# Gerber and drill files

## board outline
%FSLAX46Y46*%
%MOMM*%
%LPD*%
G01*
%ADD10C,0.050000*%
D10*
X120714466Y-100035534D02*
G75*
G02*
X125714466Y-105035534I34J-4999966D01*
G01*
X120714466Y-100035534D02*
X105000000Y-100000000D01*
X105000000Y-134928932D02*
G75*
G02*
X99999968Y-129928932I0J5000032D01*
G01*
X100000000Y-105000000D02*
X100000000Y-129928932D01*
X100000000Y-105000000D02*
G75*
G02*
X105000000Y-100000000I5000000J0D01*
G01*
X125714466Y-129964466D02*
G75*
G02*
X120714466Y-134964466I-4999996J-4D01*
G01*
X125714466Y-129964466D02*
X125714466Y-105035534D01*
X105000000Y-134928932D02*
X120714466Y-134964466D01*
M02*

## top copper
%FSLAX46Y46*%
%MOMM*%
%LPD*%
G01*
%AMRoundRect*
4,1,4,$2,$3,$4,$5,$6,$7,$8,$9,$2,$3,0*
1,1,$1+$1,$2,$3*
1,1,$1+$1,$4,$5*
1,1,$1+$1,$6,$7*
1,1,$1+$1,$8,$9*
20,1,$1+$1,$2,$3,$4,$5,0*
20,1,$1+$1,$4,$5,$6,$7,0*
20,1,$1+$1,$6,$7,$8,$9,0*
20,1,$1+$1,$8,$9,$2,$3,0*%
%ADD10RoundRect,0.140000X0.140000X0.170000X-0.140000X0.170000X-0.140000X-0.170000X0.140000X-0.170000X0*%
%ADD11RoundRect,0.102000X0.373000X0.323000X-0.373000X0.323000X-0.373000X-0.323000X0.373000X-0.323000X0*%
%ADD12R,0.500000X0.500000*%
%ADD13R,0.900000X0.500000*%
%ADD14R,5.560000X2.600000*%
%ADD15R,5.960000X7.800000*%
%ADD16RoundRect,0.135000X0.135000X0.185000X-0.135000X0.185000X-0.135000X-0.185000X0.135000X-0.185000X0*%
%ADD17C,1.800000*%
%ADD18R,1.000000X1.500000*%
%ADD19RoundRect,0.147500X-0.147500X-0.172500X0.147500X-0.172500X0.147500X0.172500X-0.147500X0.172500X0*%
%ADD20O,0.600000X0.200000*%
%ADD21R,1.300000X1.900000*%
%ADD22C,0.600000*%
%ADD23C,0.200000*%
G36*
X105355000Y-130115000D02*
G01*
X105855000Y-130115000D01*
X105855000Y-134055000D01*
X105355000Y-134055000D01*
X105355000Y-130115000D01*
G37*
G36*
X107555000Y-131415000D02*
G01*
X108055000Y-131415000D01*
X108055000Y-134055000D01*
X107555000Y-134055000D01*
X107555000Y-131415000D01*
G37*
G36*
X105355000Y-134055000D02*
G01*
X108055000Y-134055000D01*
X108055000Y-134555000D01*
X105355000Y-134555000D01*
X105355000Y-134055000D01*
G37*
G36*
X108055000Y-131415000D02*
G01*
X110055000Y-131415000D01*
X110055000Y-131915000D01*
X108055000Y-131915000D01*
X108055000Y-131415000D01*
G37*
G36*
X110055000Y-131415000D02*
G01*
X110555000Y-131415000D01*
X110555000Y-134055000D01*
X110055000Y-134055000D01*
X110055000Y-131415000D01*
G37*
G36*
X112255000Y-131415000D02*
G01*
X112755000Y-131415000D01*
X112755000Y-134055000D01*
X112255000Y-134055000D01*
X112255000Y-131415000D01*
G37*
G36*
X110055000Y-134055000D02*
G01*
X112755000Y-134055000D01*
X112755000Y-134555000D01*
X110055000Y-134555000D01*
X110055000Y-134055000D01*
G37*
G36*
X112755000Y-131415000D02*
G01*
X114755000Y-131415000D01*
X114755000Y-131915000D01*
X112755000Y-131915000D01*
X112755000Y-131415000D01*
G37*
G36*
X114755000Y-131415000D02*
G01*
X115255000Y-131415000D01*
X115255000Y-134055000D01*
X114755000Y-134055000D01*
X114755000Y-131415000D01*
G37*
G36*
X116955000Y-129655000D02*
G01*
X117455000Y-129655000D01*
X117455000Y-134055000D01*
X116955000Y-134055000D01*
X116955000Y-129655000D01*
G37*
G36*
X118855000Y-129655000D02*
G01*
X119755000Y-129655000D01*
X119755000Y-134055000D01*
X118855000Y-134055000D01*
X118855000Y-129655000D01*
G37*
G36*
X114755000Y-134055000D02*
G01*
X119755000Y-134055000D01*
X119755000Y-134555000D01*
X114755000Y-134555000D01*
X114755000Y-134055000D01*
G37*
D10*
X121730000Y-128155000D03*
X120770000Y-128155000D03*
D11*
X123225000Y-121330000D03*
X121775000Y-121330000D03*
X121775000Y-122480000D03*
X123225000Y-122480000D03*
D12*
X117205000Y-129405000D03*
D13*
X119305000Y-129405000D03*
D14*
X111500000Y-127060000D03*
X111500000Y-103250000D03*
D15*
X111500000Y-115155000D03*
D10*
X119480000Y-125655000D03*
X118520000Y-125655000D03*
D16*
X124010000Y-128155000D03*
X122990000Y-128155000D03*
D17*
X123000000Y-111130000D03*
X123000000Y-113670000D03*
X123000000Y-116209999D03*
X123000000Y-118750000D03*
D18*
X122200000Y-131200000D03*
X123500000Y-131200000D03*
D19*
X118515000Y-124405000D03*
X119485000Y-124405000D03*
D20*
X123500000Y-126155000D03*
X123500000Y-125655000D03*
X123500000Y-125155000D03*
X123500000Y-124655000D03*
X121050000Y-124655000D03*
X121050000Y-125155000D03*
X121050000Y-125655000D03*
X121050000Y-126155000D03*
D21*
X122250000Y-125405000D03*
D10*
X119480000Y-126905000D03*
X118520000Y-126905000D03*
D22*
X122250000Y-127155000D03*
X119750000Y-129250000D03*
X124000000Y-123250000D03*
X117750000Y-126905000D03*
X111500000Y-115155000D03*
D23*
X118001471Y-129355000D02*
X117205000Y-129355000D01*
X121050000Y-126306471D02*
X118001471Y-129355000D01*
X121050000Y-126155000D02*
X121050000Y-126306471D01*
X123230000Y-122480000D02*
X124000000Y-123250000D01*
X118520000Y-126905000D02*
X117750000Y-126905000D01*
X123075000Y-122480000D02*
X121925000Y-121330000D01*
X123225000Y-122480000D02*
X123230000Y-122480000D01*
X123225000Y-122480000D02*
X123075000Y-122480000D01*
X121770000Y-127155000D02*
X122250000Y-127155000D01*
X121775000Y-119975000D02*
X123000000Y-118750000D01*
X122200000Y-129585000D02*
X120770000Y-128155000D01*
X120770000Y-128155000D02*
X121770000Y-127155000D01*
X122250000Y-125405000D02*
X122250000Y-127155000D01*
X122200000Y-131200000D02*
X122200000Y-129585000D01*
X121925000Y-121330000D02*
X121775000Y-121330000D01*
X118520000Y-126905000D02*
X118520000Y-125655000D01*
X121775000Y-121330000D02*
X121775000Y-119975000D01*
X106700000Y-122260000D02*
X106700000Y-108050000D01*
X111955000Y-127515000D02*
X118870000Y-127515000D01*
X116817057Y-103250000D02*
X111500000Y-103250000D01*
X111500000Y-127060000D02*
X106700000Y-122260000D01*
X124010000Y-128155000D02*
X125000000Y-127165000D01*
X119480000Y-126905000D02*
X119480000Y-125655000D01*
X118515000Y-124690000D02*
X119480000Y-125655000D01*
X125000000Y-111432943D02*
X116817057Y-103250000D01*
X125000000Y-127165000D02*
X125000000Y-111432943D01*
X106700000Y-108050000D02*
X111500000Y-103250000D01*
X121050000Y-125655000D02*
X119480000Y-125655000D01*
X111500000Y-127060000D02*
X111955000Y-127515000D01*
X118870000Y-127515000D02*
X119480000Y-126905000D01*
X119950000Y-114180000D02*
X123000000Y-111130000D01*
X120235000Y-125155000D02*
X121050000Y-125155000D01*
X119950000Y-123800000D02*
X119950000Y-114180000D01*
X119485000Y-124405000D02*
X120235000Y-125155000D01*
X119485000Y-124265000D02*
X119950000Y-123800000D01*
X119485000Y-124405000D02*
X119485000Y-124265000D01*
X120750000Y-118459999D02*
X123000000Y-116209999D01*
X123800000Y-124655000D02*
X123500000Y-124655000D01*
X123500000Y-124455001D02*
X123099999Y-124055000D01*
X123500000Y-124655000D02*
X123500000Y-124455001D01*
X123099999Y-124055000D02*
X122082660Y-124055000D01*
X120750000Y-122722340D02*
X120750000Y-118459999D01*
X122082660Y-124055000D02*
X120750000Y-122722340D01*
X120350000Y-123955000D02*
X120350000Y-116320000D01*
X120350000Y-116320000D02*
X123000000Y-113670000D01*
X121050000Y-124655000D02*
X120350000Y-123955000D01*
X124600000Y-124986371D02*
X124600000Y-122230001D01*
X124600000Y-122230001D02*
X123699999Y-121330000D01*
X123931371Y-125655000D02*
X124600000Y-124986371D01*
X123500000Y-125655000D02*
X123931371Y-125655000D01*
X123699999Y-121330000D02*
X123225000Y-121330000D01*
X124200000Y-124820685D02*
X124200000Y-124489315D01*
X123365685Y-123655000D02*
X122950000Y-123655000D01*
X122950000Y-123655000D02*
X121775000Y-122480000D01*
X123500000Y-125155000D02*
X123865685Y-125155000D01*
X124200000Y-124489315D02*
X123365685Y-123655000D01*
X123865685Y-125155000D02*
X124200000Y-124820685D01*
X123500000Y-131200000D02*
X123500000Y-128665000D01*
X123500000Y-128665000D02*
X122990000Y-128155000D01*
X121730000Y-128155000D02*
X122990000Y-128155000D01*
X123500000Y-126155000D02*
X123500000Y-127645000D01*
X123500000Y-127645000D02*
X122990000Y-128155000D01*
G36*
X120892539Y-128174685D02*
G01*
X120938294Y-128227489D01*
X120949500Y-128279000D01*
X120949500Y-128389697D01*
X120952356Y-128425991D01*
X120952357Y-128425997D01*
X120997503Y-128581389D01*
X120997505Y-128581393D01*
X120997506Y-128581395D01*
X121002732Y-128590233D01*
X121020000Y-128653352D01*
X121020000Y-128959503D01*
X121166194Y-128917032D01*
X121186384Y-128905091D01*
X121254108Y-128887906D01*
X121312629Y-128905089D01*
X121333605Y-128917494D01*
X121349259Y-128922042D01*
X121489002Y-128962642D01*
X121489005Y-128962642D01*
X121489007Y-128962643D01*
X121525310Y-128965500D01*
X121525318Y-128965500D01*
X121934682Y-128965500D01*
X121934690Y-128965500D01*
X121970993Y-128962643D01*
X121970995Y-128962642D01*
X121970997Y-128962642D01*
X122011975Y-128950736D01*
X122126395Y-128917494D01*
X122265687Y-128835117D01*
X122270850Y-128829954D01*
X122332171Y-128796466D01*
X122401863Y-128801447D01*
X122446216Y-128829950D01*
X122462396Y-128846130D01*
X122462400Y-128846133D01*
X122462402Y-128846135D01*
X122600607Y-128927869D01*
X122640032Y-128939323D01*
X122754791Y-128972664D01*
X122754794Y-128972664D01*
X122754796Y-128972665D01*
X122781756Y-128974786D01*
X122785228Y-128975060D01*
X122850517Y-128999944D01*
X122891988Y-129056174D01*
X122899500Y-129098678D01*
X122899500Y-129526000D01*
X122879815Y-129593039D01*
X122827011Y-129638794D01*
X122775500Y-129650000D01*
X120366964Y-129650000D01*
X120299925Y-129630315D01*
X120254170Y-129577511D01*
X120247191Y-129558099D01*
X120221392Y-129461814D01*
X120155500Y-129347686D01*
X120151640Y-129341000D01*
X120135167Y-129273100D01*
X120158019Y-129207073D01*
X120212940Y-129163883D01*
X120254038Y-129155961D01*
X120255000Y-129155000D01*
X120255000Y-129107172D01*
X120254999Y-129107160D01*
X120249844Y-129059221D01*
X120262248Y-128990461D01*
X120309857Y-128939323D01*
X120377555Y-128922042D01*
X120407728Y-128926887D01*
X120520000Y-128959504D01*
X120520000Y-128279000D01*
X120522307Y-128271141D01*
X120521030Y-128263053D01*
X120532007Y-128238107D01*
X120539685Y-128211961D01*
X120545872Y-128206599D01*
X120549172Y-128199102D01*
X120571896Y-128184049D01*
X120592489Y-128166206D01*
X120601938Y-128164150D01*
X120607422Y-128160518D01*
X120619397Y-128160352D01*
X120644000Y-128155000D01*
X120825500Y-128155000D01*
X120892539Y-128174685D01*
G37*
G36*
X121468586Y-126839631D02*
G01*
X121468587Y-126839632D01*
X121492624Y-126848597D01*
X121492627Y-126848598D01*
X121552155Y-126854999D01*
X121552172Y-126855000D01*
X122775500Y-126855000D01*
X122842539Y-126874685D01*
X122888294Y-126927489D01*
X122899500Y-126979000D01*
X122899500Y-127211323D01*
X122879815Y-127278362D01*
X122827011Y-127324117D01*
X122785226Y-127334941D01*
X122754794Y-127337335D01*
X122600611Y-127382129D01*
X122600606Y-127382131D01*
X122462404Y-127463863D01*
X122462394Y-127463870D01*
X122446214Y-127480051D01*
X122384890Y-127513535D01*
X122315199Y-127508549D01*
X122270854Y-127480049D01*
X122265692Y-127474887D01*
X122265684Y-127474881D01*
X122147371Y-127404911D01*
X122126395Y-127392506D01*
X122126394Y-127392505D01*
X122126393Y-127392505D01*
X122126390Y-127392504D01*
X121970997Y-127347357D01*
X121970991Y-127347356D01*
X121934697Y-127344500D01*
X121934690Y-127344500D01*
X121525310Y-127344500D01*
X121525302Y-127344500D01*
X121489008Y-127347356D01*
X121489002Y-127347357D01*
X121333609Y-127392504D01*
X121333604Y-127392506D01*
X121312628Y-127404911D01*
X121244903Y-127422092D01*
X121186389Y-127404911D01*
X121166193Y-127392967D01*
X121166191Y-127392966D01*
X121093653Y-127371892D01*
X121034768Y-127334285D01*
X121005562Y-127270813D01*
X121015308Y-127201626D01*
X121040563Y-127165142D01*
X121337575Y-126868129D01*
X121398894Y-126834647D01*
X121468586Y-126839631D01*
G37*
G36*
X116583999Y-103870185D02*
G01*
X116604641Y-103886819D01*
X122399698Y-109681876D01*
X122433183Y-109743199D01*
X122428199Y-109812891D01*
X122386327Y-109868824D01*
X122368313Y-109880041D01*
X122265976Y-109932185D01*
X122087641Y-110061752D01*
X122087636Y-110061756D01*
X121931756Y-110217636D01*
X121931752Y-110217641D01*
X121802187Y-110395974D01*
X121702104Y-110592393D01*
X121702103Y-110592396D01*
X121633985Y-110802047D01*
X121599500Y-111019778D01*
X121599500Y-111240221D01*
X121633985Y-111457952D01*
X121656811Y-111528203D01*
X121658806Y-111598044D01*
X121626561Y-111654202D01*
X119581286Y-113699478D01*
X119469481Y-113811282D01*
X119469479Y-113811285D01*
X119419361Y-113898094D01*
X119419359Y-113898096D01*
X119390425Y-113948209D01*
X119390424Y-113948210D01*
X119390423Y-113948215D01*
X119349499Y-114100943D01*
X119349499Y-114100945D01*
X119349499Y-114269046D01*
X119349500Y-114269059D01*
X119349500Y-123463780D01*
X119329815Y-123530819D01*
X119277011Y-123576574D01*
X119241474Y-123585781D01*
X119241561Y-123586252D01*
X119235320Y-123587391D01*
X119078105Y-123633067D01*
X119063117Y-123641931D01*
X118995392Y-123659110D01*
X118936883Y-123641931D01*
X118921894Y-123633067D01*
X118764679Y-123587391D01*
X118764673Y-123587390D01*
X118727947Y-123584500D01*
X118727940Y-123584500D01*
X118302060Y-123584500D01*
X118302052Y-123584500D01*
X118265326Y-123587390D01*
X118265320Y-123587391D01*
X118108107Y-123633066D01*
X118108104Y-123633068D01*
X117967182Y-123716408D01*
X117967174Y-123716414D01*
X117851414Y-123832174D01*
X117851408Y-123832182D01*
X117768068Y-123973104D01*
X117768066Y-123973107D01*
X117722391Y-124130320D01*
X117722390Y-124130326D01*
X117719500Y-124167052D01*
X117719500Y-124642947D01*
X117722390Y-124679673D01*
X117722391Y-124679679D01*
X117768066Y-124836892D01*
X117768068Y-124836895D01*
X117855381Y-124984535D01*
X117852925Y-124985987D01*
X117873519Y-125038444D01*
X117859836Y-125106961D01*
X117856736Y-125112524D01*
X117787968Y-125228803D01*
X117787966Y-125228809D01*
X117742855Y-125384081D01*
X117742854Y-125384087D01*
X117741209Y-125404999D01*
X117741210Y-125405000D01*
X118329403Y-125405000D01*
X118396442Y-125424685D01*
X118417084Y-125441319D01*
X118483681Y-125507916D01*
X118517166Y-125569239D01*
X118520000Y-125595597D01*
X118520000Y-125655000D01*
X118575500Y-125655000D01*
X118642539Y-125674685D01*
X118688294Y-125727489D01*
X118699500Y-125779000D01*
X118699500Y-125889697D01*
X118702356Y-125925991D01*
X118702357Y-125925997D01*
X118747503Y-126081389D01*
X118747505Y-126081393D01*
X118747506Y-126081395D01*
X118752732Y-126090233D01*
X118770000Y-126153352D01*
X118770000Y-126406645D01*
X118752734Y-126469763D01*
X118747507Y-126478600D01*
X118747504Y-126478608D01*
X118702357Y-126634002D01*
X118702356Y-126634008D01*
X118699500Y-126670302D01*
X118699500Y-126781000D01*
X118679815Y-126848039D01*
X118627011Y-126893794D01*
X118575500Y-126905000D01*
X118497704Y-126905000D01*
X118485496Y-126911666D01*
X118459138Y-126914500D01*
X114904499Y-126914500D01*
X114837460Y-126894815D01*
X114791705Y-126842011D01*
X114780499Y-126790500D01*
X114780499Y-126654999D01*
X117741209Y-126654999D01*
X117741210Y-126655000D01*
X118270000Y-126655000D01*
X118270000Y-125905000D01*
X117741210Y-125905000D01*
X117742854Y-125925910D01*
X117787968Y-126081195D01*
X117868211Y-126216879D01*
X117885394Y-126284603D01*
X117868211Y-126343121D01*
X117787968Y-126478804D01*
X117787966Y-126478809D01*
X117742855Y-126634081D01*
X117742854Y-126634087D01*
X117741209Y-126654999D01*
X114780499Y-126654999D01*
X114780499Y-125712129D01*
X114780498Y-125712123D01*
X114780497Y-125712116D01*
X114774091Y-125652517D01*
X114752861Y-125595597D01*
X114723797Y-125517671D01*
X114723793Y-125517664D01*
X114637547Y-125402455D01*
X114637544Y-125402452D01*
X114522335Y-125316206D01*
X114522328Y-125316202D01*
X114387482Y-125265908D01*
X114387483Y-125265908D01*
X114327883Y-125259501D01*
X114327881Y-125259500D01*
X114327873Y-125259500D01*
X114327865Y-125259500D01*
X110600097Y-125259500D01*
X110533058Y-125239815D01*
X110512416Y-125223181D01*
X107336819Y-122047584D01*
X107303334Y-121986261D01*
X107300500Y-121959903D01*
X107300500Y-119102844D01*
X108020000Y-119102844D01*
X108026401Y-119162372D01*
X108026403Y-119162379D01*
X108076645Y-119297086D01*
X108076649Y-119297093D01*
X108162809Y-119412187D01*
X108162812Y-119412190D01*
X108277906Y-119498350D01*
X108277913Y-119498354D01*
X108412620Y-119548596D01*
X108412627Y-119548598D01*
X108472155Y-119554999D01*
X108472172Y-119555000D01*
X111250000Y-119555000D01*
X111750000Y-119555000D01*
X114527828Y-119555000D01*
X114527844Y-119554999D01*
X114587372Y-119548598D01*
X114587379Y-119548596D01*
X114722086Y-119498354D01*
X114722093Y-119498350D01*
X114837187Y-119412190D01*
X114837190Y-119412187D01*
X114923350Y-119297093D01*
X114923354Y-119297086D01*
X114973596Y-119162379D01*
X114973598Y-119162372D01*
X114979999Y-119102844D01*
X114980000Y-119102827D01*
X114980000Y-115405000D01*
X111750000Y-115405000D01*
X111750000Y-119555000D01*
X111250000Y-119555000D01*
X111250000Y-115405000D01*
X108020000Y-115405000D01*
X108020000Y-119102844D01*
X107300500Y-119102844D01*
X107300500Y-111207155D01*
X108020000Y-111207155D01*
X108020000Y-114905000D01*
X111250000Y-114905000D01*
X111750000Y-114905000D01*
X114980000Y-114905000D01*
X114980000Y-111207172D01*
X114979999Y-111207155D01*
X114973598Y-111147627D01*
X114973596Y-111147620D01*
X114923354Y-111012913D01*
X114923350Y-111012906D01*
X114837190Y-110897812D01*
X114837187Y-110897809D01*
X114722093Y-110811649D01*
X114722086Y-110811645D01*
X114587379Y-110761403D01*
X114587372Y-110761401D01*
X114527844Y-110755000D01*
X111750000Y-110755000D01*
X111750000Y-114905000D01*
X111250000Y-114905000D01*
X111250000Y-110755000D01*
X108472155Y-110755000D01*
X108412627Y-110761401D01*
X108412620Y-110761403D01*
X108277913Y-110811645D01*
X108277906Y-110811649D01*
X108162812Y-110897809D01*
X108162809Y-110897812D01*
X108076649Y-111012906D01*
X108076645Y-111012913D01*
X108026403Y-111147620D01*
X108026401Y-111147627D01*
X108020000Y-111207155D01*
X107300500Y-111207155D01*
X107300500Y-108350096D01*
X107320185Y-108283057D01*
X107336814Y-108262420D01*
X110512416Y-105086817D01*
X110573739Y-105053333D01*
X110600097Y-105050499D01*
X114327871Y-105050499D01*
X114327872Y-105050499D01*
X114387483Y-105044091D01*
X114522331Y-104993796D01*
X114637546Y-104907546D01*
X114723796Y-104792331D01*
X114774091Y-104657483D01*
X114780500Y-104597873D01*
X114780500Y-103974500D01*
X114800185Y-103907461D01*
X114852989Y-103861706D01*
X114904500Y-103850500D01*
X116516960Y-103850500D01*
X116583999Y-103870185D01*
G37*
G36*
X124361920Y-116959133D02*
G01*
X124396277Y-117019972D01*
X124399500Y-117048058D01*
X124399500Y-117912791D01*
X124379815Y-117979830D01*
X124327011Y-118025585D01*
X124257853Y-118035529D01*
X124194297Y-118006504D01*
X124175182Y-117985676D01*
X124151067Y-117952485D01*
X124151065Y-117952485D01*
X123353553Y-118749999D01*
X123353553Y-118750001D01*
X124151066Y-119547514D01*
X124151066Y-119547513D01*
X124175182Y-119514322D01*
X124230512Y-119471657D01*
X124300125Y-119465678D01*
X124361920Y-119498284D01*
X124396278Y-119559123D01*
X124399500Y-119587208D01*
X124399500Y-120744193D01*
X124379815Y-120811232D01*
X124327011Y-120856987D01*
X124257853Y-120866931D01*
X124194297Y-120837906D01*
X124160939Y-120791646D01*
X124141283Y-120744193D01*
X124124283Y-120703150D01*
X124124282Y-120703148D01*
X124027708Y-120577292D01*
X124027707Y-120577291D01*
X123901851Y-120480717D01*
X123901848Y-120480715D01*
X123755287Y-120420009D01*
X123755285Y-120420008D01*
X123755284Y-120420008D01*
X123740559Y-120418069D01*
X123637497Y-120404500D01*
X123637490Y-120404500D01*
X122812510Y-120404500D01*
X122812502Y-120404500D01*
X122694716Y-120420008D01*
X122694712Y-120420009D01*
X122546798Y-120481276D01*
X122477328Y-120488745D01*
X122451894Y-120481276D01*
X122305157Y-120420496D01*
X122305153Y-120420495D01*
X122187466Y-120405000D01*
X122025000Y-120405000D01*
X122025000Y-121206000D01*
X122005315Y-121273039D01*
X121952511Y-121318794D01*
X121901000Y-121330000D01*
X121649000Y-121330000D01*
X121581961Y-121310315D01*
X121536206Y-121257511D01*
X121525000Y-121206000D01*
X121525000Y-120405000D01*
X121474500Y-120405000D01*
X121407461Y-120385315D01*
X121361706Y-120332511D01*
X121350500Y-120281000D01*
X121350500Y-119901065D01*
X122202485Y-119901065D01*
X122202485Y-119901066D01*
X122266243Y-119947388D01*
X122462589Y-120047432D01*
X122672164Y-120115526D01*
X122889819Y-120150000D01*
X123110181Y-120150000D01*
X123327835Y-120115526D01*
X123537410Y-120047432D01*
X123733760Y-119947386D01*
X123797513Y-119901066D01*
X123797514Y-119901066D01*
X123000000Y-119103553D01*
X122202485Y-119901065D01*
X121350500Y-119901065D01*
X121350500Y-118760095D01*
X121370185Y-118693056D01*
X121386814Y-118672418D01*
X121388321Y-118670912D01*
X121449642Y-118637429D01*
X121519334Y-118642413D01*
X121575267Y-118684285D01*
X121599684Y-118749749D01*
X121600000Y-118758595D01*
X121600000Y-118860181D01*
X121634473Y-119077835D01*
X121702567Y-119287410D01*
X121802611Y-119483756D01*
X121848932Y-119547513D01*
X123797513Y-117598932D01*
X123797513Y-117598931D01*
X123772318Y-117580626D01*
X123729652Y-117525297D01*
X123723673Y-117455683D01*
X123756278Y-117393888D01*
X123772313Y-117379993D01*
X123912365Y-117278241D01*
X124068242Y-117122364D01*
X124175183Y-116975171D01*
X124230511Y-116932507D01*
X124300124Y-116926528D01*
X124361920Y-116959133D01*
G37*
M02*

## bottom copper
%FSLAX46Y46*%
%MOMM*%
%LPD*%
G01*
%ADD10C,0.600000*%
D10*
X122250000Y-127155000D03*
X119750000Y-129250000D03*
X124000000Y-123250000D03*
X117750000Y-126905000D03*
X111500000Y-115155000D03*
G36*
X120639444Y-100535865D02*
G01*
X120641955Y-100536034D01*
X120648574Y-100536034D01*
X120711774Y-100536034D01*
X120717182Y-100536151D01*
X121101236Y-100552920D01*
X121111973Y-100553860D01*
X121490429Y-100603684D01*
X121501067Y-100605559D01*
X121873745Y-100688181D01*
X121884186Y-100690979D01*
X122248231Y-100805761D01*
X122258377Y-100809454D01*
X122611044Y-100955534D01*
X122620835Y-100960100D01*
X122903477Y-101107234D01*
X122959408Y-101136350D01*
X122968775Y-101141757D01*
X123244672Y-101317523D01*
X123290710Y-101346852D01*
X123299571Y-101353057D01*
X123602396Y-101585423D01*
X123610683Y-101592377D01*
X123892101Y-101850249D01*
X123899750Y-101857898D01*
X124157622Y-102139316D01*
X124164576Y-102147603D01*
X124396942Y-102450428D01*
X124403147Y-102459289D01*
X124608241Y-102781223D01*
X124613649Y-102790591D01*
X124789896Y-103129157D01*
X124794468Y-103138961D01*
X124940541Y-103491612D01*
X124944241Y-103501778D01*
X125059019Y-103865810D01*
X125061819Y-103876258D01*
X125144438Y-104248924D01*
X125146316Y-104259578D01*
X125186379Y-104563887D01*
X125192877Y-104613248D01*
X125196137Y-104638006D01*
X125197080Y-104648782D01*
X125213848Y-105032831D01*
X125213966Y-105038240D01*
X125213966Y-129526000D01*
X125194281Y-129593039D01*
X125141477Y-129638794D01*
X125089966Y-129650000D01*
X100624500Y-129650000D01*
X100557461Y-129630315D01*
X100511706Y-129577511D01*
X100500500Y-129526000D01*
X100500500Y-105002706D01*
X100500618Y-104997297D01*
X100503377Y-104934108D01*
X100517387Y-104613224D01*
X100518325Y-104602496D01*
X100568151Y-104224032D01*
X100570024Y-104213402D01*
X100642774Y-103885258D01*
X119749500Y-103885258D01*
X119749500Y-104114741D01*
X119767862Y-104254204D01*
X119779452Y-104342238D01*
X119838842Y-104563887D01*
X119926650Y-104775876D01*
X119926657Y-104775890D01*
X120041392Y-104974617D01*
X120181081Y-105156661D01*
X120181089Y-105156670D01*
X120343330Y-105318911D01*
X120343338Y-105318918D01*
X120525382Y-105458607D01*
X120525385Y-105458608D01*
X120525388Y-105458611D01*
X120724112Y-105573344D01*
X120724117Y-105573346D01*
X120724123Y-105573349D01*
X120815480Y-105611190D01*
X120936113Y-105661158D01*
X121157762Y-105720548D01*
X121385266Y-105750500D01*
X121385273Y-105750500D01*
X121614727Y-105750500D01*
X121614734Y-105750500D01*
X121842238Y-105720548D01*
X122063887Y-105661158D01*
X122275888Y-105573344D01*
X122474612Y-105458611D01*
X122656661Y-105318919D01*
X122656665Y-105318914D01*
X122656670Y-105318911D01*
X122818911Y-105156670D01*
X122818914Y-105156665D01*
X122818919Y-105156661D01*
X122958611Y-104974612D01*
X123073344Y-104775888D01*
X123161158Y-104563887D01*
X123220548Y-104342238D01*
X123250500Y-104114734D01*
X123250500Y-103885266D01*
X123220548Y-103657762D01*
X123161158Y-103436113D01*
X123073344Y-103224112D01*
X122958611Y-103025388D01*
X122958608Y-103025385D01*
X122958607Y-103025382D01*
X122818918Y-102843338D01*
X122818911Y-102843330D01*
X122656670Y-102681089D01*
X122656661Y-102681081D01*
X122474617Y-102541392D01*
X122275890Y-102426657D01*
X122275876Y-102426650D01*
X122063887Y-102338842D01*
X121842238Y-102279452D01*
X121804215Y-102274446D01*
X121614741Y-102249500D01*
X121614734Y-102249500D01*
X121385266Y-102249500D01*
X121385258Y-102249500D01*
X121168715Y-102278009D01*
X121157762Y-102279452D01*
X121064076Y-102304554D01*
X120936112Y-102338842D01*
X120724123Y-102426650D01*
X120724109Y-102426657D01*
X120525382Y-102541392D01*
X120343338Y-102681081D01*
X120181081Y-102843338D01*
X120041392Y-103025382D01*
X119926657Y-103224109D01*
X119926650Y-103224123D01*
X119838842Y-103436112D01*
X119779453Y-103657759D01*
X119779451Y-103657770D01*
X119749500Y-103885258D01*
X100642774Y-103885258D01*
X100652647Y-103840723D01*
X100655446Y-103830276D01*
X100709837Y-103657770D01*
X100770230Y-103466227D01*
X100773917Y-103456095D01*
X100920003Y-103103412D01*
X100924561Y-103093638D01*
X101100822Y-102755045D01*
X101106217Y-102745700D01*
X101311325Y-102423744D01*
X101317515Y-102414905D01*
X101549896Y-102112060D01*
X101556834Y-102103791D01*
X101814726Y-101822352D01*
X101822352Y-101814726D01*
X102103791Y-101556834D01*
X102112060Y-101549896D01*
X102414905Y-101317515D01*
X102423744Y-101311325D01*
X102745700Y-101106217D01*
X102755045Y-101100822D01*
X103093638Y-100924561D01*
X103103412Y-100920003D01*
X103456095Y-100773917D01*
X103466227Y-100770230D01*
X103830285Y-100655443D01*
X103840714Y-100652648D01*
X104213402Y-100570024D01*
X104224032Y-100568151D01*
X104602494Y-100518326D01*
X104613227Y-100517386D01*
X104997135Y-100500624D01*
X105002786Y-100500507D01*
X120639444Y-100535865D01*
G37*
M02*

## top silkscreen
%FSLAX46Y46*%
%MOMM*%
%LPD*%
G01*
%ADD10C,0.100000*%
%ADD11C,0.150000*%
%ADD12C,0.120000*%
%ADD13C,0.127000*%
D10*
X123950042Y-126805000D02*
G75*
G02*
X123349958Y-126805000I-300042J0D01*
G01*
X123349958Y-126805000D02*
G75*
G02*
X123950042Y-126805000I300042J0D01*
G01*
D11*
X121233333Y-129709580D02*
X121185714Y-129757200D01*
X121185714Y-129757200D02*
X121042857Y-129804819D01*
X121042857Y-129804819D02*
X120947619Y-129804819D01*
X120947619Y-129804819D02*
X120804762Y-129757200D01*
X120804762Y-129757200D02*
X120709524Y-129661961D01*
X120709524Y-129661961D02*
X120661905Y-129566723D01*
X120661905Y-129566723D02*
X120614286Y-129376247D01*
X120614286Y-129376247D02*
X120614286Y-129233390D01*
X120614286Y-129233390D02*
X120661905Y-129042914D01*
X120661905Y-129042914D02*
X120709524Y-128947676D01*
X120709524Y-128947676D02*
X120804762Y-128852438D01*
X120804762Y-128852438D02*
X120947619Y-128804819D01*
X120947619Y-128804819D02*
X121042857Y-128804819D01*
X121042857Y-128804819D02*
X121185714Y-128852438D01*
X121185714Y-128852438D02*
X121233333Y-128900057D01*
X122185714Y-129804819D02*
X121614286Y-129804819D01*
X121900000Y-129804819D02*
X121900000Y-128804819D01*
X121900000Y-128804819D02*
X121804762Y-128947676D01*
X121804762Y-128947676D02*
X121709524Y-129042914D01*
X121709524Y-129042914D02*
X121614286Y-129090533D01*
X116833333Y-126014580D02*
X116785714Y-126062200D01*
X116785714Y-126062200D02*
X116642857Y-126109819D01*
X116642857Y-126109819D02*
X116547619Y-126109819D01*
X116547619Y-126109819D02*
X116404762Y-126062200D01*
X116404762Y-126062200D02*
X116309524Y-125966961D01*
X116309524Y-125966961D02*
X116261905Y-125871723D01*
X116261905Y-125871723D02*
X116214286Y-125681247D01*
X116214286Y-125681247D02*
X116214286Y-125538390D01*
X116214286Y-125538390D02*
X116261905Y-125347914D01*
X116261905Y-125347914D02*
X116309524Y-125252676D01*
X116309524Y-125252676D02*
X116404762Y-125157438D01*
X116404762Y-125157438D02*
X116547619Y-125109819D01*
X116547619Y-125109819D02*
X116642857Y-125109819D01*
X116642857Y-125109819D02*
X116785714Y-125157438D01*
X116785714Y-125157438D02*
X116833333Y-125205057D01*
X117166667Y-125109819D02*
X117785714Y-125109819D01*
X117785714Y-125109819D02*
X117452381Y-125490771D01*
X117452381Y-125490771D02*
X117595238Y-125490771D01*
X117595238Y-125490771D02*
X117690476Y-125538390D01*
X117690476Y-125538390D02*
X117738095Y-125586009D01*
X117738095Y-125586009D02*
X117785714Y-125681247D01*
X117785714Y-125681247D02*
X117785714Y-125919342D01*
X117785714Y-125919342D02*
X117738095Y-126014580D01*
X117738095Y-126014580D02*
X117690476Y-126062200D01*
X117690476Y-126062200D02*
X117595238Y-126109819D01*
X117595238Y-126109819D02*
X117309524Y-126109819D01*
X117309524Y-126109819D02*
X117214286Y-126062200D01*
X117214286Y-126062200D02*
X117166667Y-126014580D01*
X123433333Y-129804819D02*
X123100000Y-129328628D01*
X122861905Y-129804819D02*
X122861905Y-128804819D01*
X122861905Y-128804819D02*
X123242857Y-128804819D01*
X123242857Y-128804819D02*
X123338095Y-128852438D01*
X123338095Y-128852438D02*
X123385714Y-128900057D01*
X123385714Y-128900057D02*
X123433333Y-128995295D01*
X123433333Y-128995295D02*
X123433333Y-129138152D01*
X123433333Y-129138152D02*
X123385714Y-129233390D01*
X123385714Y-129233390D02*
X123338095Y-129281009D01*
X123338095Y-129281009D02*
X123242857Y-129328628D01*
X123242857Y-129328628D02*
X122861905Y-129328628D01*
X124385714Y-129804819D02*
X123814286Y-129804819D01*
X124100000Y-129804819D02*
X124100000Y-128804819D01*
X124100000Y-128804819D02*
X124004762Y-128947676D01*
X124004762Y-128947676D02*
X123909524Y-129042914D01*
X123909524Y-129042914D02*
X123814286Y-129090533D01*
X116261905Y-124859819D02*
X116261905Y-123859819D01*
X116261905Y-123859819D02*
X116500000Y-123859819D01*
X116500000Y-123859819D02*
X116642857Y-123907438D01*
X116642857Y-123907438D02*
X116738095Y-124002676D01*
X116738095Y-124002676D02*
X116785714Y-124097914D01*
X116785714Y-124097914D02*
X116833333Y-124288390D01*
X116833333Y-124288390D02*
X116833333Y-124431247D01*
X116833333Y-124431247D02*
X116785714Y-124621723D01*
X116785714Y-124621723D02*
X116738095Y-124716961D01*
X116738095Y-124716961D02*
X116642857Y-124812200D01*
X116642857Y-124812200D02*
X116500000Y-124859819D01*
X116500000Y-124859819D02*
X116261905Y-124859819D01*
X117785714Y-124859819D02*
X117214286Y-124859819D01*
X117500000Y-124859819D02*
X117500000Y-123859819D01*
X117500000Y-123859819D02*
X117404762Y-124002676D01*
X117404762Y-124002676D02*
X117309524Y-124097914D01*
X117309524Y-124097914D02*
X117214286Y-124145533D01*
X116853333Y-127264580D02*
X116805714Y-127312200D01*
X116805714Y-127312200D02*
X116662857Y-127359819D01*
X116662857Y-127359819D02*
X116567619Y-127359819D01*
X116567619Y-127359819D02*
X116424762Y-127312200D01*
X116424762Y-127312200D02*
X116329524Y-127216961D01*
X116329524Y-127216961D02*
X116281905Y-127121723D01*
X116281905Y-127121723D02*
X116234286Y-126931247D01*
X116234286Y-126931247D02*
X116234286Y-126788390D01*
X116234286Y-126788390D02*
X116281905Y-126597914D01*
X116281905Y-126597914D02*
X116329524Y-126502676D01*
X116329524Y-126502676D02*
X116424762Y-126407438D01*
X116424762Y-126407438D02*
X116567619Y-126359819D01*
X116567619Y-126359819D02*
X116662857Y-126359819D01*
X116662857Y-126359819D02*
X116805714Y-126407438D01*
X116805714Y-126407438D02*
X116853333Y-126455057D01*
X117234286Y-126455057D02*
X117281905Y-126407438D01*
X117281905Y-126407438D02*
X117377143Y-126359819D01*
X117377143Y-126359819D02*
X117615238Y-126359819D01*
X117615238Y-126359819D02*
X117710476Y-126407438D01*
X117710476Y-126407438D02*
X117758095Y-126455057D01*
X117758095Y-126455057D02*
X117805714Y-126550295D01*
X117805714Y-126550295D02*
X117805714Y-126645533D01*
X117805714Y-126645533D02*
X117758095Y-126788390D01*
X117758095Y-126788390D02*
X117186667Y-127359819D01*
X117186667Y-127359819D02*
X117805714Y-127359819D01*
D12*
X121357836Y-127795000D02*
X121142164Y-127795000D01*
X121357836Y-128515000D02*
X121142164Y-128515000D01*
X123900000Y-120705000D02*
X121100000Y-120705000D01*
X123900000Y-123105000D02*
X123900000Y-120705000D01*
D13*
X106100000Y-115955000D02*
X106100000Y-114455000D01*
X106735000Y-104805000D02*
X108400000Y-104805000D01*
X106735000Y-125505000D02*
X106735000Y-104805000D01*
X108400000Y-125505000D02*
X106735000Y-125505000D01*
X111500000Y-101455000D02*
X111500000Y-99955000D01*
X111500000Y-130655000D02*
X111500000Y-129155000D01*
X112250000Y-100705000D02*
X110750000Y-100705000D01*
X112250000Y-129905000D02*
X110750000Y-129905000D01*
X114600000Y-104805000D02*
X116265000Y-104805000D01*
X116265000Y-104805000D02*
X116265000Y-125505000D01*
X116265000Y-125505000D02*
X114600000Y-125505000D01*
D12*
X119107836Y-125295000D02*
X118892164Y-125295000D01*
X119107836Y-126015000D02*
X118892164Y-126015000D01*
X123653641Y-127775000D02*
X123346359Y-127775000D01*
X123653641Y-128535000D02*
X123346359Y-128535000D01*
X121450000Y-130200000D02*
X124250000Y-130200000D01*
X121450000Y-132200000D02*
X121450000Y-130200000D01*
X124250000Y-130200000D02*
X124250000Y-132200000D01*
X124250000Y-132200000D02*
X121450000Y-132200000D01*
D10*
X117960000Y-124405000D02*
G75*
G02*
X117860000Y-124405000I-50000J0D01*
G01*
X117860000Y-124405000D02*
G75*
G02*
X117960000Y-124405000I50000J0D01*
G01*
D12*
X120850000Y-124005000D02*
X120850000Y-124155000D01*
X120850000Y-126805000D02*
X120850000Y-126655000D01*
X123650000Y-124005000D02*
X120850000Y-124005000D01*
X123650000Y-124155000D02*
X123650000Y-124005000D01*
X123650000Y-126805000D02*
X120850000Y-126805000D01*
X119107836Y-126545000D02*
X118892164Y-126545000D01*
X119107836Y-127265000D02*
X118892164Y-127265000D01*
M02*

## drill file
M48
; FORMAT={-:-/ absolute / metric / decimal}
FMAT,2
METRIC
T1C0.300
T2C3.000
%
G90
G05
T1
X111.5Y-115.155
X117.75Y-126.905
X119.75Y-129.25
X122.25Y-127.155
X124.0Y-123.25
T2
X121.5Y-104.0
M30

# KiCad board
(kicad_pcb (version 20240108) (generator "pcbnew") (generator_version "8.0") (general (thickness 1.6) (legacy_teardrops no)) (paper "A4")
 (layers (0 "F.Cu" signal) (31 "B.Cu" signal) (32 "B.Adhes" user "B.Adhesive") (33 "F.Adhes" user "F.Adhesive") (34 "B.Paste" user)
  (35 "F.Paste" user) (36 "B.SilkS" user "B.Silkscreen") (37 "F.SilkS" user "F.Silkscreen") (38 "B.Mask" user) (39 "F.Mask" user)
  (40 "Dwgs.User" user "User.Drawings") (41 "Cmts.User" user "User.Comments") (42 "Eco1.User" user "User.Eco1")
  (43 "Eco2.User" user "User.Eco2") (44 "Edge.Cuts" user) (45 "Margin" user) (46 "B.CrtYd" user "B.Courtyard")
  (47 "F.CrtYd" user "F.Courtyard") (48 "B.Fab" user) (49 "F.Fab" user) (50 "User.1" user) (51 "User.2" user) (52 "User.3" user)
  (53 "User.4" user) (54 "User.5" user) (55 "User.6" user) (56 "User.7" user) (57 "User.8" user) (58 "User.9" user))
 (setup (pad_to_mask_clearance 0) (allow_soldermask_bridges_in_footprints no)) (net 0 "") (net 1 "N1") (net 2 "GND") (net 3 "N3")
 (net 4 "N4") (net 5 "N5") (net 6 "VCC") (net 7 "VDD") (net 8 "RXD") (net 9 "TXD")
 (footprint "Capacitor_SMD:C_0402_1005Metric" (layer "F.Cu") (at 121.25 128.155 180)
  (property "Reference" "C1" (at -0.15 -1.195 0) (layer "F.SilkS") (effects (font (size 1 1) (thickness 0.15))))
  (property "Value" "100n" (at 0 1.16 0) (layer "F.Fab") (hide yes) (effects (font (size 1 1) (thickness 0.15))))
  (fp_line (start -0.107836 0.36) (end 0.107836 0.36) (stroke (width 0.12) (type solid)) (layer "F.SilkS"))
  (fp_line (start -0.107836 -0.36) (end 0.107836 -0.36) (stroke (width 0.12) (type solid)) (layer "F.SilkS"))
  (pad "1" smd roundrect (at -0.48 0 180) (size 0.56 0.62) (layers "F.Cu" "F.Paste" "F.Mask") (roundrect_rratio 0.25) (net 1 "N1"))
  (pad "2" smd roundrect (at 0.48 0 180) (size 0.56 0.62) (layers "F.Cu" "F.Paste" "F.Mask") (roundrect_rratio 0.25) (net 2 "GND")))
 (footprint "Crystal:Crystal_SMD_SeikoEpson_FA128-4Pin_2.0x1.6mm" (layer "F.Cu") (at 122.5 121.905 180)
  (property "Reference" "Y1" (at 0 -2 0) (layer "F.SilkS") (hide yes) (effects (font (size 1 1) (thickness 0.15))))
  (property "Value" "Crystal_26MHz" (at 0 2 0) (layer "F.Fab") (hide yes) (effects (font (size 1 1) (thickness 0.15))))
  (fp_line (start -1.4 1.2) (end 1.4 1.2) (stroke (width 0.12) (type solid)) (layer "F.SilkS"))
  (fp_line (start -1.4 -1.2) (end -1.4 1.2) (stroke (width 0.12) (type solid)) (layer "F.SilkS"))
  (pad "1" smd roundrect (at -0.725 0.575 180) (size 0.95 0.85) (layers "F.Cu" "F.Paste" "F.Mask") (roundrect_rratio 0.12) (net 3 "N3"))
  (pad "2" smd roundrect (at 0.725 0.575 180) (size 0.95 0.85) (layers "F.Cu" "F.Paste" "F.Mask") (roundrect_rratio 0.12) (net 2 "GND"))
  (pad "3" smd roundrect (at 0.725 -0.575 180) (size 0.95 0.85) (layers "F.Cu" "F.Paste" "F.Mask") (roundrect_rratio 0.12) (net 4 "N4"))
  (pad "4" smd roundrect (at -0.725 -0.575 180) (size 0.95 0.85) (layers "F.Cu" "F.Paste" "F.Mask") (roundrect_rratio 0.12) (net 2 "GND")))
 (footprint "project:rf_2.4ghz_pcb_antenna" (layer "F.Cu") (at 120.255 134.855 180)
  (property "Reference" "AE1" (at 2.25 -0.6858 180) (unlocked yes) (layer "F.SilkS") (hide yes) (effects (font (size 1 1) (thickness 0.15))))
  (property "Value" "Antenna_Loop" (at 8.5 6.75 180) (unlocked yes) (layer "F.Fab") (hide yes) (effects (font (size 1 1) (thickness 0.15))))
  (fp_rect (start 14.4 0.8) (end 14.9 4.74) (stroke (width 0) (type solid)) (fill solid) (layer "F.Cu"))
  (fp_rect (start 12.2 0.8) (end 12.7 3.44) (stroke (width 0) (type default)) (fill solid) (layer "F.Cu"))
  (fp_rect (start 12.2 0.3) (end 14.9 0.8) (stroke (width 0) (type default)) (fill solid) (layer "F.Cu"))
  (fp_rect (start 10.2 2.94) (end 12.2 3.44) (stroke (width 0) (type default)) (fill solid) (layer "F.Cu"))
  (fp_rect (start 9.7 0.8) (end 10.2 3.44) (stroke (width 0) (type default)) (fill solid) (layer "F.Cu"))
  (fp_rect (start 7.5 0.8) (end 8 3.44) (stroke (width 0) (type default)) (fill solid) (layer "F.Cu"))
  (fp_rect (start 7.5 0.3) (end 10.2 0.8) (stroke (width 0) (type default)) (fill solid) (layer "F.Cu"))
  (fp_rect (start 5.5 2.94) (end 7.5 3.44) (stroke (width 0) (type default)) (fill solid) (layer "F.Cu"))
  (fp_rect (start 5 0.8) (end 5.5 3.44) (stroke (width 0) (type default)) (fill solid) (layer "F.Cu"))
  (fp_rect (start 2.8 0.8) (end 3.3 5.2) (stroke (width 0) (type default)) (fill solid) (layer "F.Cu"))
  (fp_rect (start 0.5 0.8) (end 1.4 5.2) (stroke (width 0) (type solid)) (fill solid) (layer "F.Cu"))
  (fp_rect (start 0.5 0.3) (end 5.5 0.8) (stroke (width 0) (type default)) (fill solid) (layer "F.Cu"))
  (pad "1" smd rect (at 3.05 5.45 180) (size 0.5 0.5) (layers "F.Cu" "F.Paste" "F.Mask") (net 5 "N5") (solder_mask_margin 0.102))
  (pad "2" smd rect (at 0.95 5.45 270) (size 0.5 0.9) (layers "F.Cu" "F.Paste" "F.Mask") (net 2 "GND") (solder_mask_margin 0.102))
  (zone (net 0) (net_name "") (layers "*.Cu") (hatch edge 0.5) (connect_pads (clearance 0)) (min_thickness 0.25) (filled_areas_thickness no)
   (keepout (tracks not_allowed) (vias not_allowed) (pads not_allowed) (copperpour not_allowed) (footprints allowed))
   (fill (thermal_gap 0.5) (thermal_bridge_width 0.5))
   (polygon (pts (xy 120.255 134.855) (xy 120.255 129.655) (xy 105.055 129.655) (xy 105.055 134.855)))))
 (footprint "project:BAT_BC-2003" (layer "F.Cu") (at 111.5 115.155 90)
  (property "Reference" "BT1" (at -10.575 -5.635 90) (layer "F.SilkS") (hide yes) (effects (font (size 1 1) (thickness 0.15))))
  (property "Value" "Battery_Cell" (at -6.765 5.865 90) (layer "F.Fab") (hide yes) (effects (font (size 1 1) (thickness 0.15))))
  (fp_line (start -0.8 -5.4) (end 0.7 -5.4) (stroke (width 0.127) (type solid)) (layer "F.SilkS"))
  (fp_line (start 10.35 -4.765) (end 10.35 -3.1) (stroke (width 0.127) (type solid)) (layer "F.SilkS"))
  (fp_line (start -10.35 -4.765) (end 10.35 -4.765) (stroke (width 0.127) (type solid)) (layer "F.SilkS"))
  (fp_line (start -10.35 -3.1) (end -10.35 -4.765) (stroke (width 0.127) (type solid)) (layer "F.SilkS"))
  (fp_line (start 13.7 0) (end 15.2 0) (stroke (width 0.127) (type solid)) (layer "F.SilkS"))
  (fp_line (start -15.5 0) (end -14 0) (stroke (width 0.127) (type solid)) (layer "F.SilkS"))
  (fp_line (start 14.45 0.75) (end 14.45 -0.75) (stroke (width 0.127) (type solid)) (layer "F.SilkS"))
  (fp_line (start -14.75 0.75) (end -14.75 -0.75) (stroke (width 0.127) (type solid)) (layer "F.SilkS"))
  (fp_line (start 10.35 3.1) (end 10.35 4.765) (stroke (width 0.127) (type solid)) (layer "F.SilkS"))
  (fp_line (start 10.35 4.765) (end -10.35 4.765) (stroke (width 0.127) (type solid)) (layer "F.SilkS"))
  (fp_line (start -10.35 4.765) (end -10.35 3.1) (stroke (width 0.127) (type solid)) (layer "F.SilkS"))
  (pad "1" smd rect (at -11.905 0 90) (size 2.6 5.56) (layers "F.Cu" "F.Paste" "F.Mask") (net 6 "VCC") (solder_mask_margin 0.102))
  (pad "1" smd rect (at 11.905 0 90) (size 2.6 5.56) (layers "F.Cu" "F.Paste" "F.Mask") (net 6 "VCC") (solder_mask_margin 0.102))
  (pad "2" smd rect (at 0 0 90) (size 7.8 5.96) (layers "F.Cu" "F.Mask") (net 2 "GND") (solder_mask_margin 0.102)))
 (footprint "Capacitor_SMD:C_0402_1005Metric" (layer "F.Cu") (at 119 125.655 180)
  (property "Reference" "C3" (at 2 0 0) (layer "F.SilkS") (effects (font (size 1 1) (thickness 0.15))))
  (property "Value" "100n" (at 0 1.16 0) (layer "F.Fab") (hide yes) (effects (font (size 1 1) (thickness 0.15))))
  (fp_line (start -0.107836 0.36) (end 0.107836 0.36) (stroke (width 0.12) (type solid)) (layer "F.SilkS"))
  (fp_line (start -0.107836 -0.36) (end 0.107836 -0.36) (stroke (width 0.12) (type solid)) (layer "F.SilkS"))
  (pad "1" smd roundrect (at -0.48 0 180) (size 0.56 0.62) (layers "F.Cu" "F.Paste" "F.Mask") (roundrect_rratio 0.25) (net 6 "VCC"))
  (pad "2" smd roundrect (at 0.48 0 180) (size 0.56 0.62) (layers "F.Cu" "F.Paste" "F.Mask") (roundrect_rratio 0.25) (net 2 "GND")))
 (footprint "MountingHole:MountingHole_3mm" (layer "F.Cu") (at 121.5 104)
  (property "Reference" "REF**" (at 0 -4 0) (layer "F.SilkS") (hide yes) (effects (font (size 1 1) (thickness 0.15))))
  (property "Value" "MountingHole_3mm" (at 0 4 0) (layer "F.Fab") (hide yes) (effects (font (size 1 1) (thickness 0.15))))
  (pad "" np_thru_hole circle (at 0 0) (size 3 3) (drill 3) (layers "*.Cu" "*.Mask")))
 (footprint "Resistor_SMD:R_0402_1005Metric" (layer "F.Cu") (at 123.5 128.155 180)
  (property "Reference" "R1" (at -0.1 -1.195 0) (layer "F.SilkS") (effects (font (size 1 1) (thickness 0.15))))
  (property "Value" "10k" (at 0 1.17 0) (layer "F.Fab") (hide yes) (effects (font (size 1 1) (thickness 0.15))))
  (fp_line (start -0.153641 0.38) (end 0.153641 0.38) (stroke (width 0.12) (type solid)) (layer "F.SilkS"))
  (fp_line (start -0.153641 -0.38) (end 0.153641 -0.38) (stroke (width 0.12) (type solid)) (layer "F.SilkS"))
  (pad "1" smd roundrect (at -0.51 0 180) (size 0.54 0.64) (layers "F.Cu" "F.Paste" "F.Mask") (roundrect_rratio 0.25) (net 6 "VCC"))
  (pad "2" smd roundrect (at 0.51 0 180) (size 0.54 0.64) (layers "F.Cu" "F.Paste" "F.Mask") (roundrect_rratio 0.25) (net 1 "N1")))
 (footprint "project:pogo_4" (layer "F.Cu") (at 123 111.13 -90)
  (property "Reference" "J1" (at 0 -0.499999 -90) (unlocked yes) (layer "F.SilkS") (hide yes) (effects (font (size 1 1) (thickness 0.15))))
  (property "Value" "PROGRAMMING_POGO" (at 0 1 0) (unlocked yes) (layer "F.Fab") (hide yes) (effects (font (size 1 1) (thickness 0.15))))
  (pad "1" smd circle (at 0 0 270) (size 1.8 1.8) (layers "F.Cu" "F.Paste" "F.Mask") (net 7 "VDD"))
  (pad "2" smd circle (at 2.54 0 270) (size 1.8 1.8) (layers "F.Cu" "F.Paste" "F.Mask") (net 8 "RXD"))
  (pad "3" smd circle (at 5.079999 0 270) (size 1.8 1.8) (layers "F.Cu" "F.Paste" "F.Mask") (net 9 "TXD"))
  (pad "4" smd circle (at 7.62 0 270) (size 1.8 1.8) (layers "F.Cu" "F.Paste" "F.Mask") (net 2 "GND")))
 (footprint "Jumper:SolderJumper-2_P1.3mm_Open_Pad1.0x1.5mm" (layer "F.Cu") (at 122.85 131.2)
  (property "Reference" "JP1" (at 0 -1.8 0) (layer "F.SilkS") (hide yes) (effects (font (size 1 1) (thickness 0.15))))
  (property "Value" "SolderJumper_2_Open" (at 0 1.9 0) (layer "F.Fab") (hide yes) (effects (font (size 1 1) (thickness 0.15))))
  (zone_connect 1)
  (fp_line (start -1.4 -1) (end 1.4 -1) (stroke (width 0.12) (type solid)) (layer "F.SilkS"))
  (fp_line (start -1.4 1) (end -1.4 -1) (stroke (width 0.12) (type solid)) (layer "F.SilkS"))
  (fp_line (start 1.4 -1) (end 1.4 1) (stroke (width 0.12) (type solid)) (layer "F.SilkS"))
  (fp_line (start 1.4 1) (end -1.4 1) (stroke (width 0.12) (type solid)) (layer "F.SilkS"))
  (pad "1" smd rect (at -0.65 0) (size 1 1.5) (layers "F.Cu" "F.Mask") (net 2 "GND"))
  (pad "2" smd rect (at 0.65 0) (size 1 1.5) (layers "F.Cu" "F.Mask") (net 1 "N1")))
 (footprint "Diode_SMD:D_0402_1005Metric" (layer "F.Cu") (at 119 124.405)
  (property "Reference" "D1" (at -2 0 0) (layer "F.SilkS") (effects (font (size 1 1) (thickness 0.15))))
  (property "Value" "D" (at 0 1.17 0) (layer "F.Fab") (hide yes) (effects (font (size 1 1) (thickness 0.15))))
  (fp_circle (center -1.09 0) (end -1.04 0) (stroke (width 0.1) (type solid)) (fill none) (layer "F.SilkS"))
  (pad "1" smd roundrect (at -0.485 0) (size 0.59 0.64) (layers "F.Cu" "F.Paste" "F.Mask") (roundrect_rratio 0.25) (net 6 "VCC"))
  (pad "2" smd roundrect (at 0.485 0) (size 0.59 0.64) (layers "F.Cu" "F.Paste" "F.Mask") (roundrect_rratio 0.25) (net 7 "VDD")))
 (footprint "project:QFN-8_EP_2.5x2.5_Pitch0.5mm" (layer "F.Cu") (at 122.25 125.405 180)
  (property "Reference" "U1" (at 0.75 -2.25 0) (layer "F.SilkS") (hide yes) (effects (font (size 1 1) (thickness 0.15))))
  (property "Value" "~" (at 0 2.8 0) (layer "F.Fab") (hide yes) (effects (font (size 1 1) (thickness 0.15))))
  (fp_line (start 1.4 1.4) (end 1.4 1.25) (stroke (width 0.12) (type default)) (layer "F.SilkS"))
  (fp_line (start 1.4 -1.4) (end 1.4 -1.25) (stroke (width 0.12) (type default)) (layer "F.SilkS"))
  (fp_line (start -1.4 1.4) (end 1.4 1.4) (stroke (width 0.12) (type default)) (layer "F.SilkS"))
  (fp_line (start -1.4 1.25) (end -1.4 1.4) (stroke (width 0.12) (type default)) (layer "F.SilkS"))
  (fp_line (start -1.4 -1.4) (end 1.4 -1.4) (stroke (width 0.12) (type default)) (layer "F.SilkS"))
  (pad "" smd rect (at -0.4875 -0.7125 180) (size 0.000001 0.150001) (layers "F.Paste") (thermal_bridge_angle 45))
  (pad "" smd rect (at -0.4875 -0.2375 180) (size 0.000001 0.150001) (layers "F.Paste") (thermal_bridge_angle 45))
  (pad "" smd rect (at -0.4875 0.2375 180) (size 0.000001 0.150001) (layers "F.Paste") (thermal_bridge_angle 45))
  (pad "" smd rect (at -0.4875 0.7125 180) (size 0.000001 0.150001) (layers "F.Paste") (thermal_bridge_angle 45))
  (pad "" smd rect (at -0.1625 -0.7125 180) (size 0.000001 0.150001) (layers "F.Paste") (thermal_bridge_angle 45))
  (pad "" smd rect (at -0.1625 -0.2375 180) (size 0.000001 0.150001) (layers "F.Paste") (thermal_bridge_angle 45))
  (pad "" smd rect (at -0.1625 0.2375 180) (size 0.000001 0.150001) (layers "F.Paste") (thermal_bridge_angle 45))
  (pad "" smd rect (at -0.1625 0.7125 180) (size 0.000001 0.150001) (layers "F.Paste") (thermal_bridge_angle 45))
  (pad "" smd rect (at 0.1625 -0.7125 180) (size 0.000001 0.150001) (layers "F.Paste") (thermal_bridge_angle 45))
  (pad "" smd rect (at 0.1625 -0.2375 180) (size 0.000001 0.150001) (layers "F.Paste") (thermal_bridge_angle 45))
  (pad "" smd rect (at 0.1625 0.2375 180) (size 0.000001 0.150001) (layers "F.Paste") (thermal_bridge_angle 45))
  (pad "" smd rect (at 0.1625 0.7125 180) (size 0.000001 0.150001) (layers "F.Paste") (thermal_bridge_angle 45))
  (pad "" smd rect (at 0.4875 -0.7125 180) (size 0.000001 0.150001) (layers "F.Paste") (thermal_bridge_angle 45))
  (pad "" smd rect (at 0.4875 -0.2375 180) (size 0.000001 0.150001) (layers "F.Paste") (thermal_bridge_angle 45))
  (pad "" smd rect (at 0.4875 0.2375 180) (size 0.000001 0.150001) (layers "F.Paste") (thermal_bridge_angle 45))
  (pad "" smd rect (at 0.4875 0.7125 180) (size 0.000001 0.150001) (layers "F.Paste") (thermal_bridge_angle 45))
  (pad "1" smd oval (at -1.25 -0.75 270) (size 0.2 0.6) (layers "F.Cu" "F.Paste" "F.Mask") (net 1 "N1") (thermal_bridge_angle 45))
  (pad "2" smd oval (at -1.25 -0.25 270) (size 0.2 0.6) (layers "F.Cu" "F.Paste" "F.Mask") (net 3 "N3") (thermal_bridge_angle 45))
  (pad "3" smd oval (at -1.25 0.25 270) (size 0.2 0.6) (layers "F.Cu" "F.Paste" "F.Mask") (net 4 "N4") (thermal_bridge_angle 45))
  (pad "4" smd oval (at -1.25 0.75 270) (size 0.2 0.6) (layers "F.Cu" "F.Paste" "F.Mask") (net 9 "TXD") (thermal_bridge_angle 45))
  (pad "5" smd oval (at 1.2 0.75 270) (size 0.2 0.6) (layers "F.Cu" "F.Paste" "F.Mask") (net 8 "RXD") (thermal_bridge_angle 45))
  (pad "6" smd oval (at 1.2 0.25 270) (size 0.2 0.6) (layers "F.Cu" "F.Paste" "F.Mask") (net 7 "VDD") (thermal_bridge_angle 45))
  (pad "7" smd oval (at 1.2 -0.25 270) (size 0.2 0.6) (layers "F.Cu" "F.Paste" "F.Mask") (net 6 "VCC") (thermal_bridge_angle 45))
  (pad "8" smd oval (at 1.2 -0.75 270) (size 0.2 0.6) (layers "F.Cu" "F.Paste" "F.Mask") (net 5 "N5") (thermal_bridge_angle 45))
  (pad "9" smd rect (at 0 0 180) (size 1.3 1.9) (layers "F.Cu" "F.Mask") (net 2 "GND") (thermal_bridge_angle 45)))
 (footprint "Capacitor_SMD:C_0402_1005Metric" (layer "F.Cu") (at 119 126.905 180)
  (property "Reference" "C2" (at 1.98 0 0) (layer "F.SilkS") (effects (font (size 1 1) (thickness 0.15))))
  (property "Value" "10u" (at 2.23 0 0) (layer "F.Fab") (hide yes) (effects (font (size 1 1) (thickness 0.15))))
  (fp_line (start -0.107836 0.36) (end 0.107836 0.36) (stroke (width 0.12) (type solid)) (layer "F.SilkS"))
  (fp_line (start -0.107836 -0.36) (end 0.107836 -0.36) (stroke (width 0.12) (type solid)) (layer "F.SilkS"))
  (pad "1" smd roundrect (at -0.48 0 180) (size 0.56 0.62) (layers "F.Cu" "F.Paste" "F.Mask") (roundrect_rratio 0.25) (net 6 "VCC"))
  (pad "2" smd roundrect (at 0.48 0 180) (size 0.56 0.62) (layers "F.Cu" "F.Paste" "F.Mask") (roundrect_rratio 0.25) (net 2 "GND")))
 (gr_circle (center 123.65 126.805) (end 123.95 126.8) (stroke (width 0.1) (type default)) (fill none) (layer "F.SilkS"))
 (gr_arc (start 120.714466 100.035534) (mid 124.25 101.5) (end 125.714466 105.035534) (stroke (width 0.05) (type default))
  (layer "Edge.Cuts"))
 (gr_line (start 120.714466 100.035534) (end 105 100) (stroke (width 0.05) (type default)) (layer "Edge.Cuts"))
 (gr_arc (start 105 134.928932) (mid 101.464465 133.464466) (end 100 129.928932) (stroke (width 0.05) (type default)) (layer "Edge.Cuts"))
 (gr_line (start 100 105) (end 100 129.928932) (stroke (width 0.05) (type default)) (layer "Edge.Cuts"))
 (gr_arc (start 100 105) (mid 101.464466 101.464466) (end 105 100) (stroke (width 0.05) (type default)) (layer "Edge.Cuts"))
 (gr_arc (start 125.714466 129.964466) (mid 124.25 133.5) (end 120.714466 134.964466) (stroke (width 0.05) (type default))
  (layer "Edge.Cuts"))
 (gr_line (start 125.714466 129.964466) (end 125.714466 105.035534) (stroke (width 0.05) (type default)) (layer "Edge.Cuts"))
 (gr_line (start 105 134.928932) (end 120.714466 134.964466) (stroke (width 0.05) (type default)) (layer "Edge.Cuts"))
 (segment (start 118.001471 129.355) (end 117.205 129.355) (width 0.2) (layer "F.Cu") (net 5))
 (segment (start 121.05 126.306471) (end 118.001471 129.355) (width 0.2) (layer "F.Cu") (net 5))
 (segment (start 121.05 126.155) (end 121.05 126.306471) (width 0.2) (layer "F.Cu") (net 5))
 (segment (start 123.23 122.48) (end 124 123.25) (width 0.2) (layer "F.Cu") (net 2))
 (segment (start 118.52 126.905) (end 117.75 126.905) (width 0.2) (layer "F.Cu") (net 2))
 (segment (start 123.075 122.48) (end 121.925 121.33) (width 0.2) (layer "F.Cu") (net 2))
 (segment (start 123.225 122.48) (end 123.23 122.48) (width 0.2) (layer "F.Cu") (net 2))
 (segment (start 123.225 122.48) (end 123.075 122.48) (width 0.2) (layer "F.Cu") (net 2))
 (segment (start 121.77 127.155) (end 122.25 127.155) (width 0.2) (layer "F.Cu") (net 2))
 (segment (start 121.775 119.975) (end 123 118.75) (width 0.2) (layer "F.Cu") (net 2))
 (segment (start 122.2 129.585) (end 120.77 128.155) (width 0.2) (layer "F.Cu") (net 2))
 (segment (start 120.77 128.155) (end 121.77 127.155) (width 0.2) (layer "F.Cu") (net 2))
 (segment (start 122.25 125.405) (end 122.25 127.155) (width 0.2) (layer "F.Cu") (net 2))
 (segment (start 122.2 131.2) (end 122.2 129.585) (width 0.2) (layer "F.Cu") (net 2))
 (segment (start 121.925 121.33) (end 121.775 121.33) (width 0.2) (layer "F.Cu") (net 2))
 (segment (start 118.52 126.905) (end 118.52 125.655) (width 0.2) (layer "F.Cu") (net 2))
 (segment (start 121.775 121.33) (end 121.775 119.975) (width 0.2) (layer "F.Cu") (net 2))
 (via (at 122.25 127.155) (size 0.6) (drill 0.3) (layers "F.Cu" "B.Cu") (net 2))
 (via (at 119.75 129.25) (size 0.6) (drill 0.3) (layers "F.Cu" "B.Cu") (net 2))
 (via (at 124 123.25) (size 0.6) (drill 0.3) (layers "F.Cu" "B.Cu") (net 2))
 (via (at 117.75 126.905) (size 0.6) (drill 0.3) (layers "F.Cu" "B.Cu") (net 2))
 (via (at 111.5 115.155) (size 0.6) (drill 0.3) (layers "F.Cu" "B.Cu") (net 2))
 (segment (start 106.7 122.26) (end 106.7 108.05) (width 0.2) (layer "F.Cu") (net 6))
 (segment (start 111.955 127.515) (end 118.87 127.515) (width 0.2) (layer "F.Cu") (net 6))
 (segment (start 116.817057 103.25) (end 111.5 103.25) (width 0.2) (layer "F.Cu") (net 6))
 (segment (start 111.5 127.06) (end 106.7 122.26) (width 0.2) (layer "F.Cu") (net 6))
 (segment (start 124.01 128.155) (end 125 127.165) (width 0.2) (layer "F.Cu") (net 6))
 (segment (start 119.48 126.905) (end 119.48 125.655) (width 0.2) (layer "F.Cu") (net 6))
 (segment (start 118.515 124.69) (end 119.48 125.655) (width 0.2) (layer "F.Cu") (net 6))
 (segment (start 125 111.432943) (end 116.817057 103.25) (width 0.2) (layer "F.Cu") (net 6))
 (segment (start 125 127.165) (end 125 111.432943) (width 0.2) (layer "F.Cu") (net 6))
 (segment (start 106.7 108.05) (end 111.5 103.25) (width 0.2) (layer "F.Cu") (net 6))
 (segment (start 121.05 125.655) (end 119.48 125.655) (width 0.2) (layer "F.Cu") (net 6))
 (segment (start 111.5 127.06) (end 111.955 127.515) (width 0.2) (layer "F.Cu") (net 6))
 (segment (start 118.87 127.515) (end 119.48 126.905) (width 0.2) (layer "F.Cu") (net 6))
 (segment (start 119.95 114.18) (end 123 111.13) (width 0.2) (layer "F.Cu") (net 7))
 (segment (start 120.235 125.155) (end 121.05 125.155) (width 0.2) (layer "F.Cu") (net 7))
 (segment (start 119.95 123.8) (end 119.95 114.18) (width 0.2) (layer "F.Cu") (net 7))
 (segment (start 119.485 124.405) (end 120.235 125.155) (width 0.2) (layer "F.Cu") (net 7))
 (segment (start 119.485 124.265) (end 119.95 123.8) (width 0.2) (layer "F.Cu") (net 7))
 (segment (start 119.485 124.405) (end 119.485 124.265) (width 0.2) (layer "F.Cu") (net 7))
 (segment (start 120.75 118.459999) (end 123 116.209999) (width 0.2) (layer "F.Cu") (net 9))
 (segment (start 123.8 124.655) (end 123.5 124.655) (width 0.2) (layer "F.Cu") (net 9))
 (segment (start 123.5 124.455001) (end 123.099999 124.055) (width 0.2) (layer "F.Cu") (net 9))
 (segment (start 123.5 124.655) (end 123.5 124.455001) (width 0.2) (layer "F.Cu") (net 9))
 (segment (start 123.099999 124.055) (end 122.08266 124.055) (width 0.2) (layer "F.Cu") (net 9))
 (segment (start 120.75 122.72234) (end 120.75 118.459999) (width 0.2) (layer "F.Cu") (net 9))
 (segment (start 122.08266 124.055) (end 120.75 122.72234) (width 0.2) (layer "F.Cu") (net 9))
 (segment (start 120.35 123.955) (end 120.35 116.32) (width 0.2) (layer "F.Cu") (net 8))
 (segment (start 120.35 116.32) (end 123 113.67) (width 0.2) (layer "F.Cu") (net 8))
 (segment (start 121.05 124.655) (end 120.35 123.955) (width 0.2) (layer "F.Cu") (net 8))
 (segment (start 124.6 124.986371) (end 124.6 122.230001) (width 0.2) (layer "F.Cu") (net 3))
 (segment (start 124.6 122.230001) (end 123.699999 121.33) (width 0.2) (layer "F.Cu") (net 3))
 (segment (start 123.931371 125.655) (end 124.6 124.986371) (width 0.2) (layer "F.Cu") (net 3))
 (segment (start 123.5 125.655) (end 123.931371 125.655) (width 0.2) (layer "F.Cu") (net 3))
 (segment (start 123.699999 121.33) (end 123.225 121.33) (width 0.2) (layer "F.Cu") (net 3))
 (segment (start 124.2 124.820685) (end 124.2 124.489315) (width 0.2) (layer "F.Cu") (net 4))
 (segment (start 123.365685 123.655) (end 122.95 123.655) (width 0.2) (layer "F.Cu") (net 4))
 (segment (start 122.95 123.655) (end 121.775 122.48) (width 0.2) (layer "F.Cu") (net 4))
 (segment (start 123.5 125.155) (end 123.865685 125.155) (width 0.2) (layer "F.Cu") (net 4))
 (segment (start 124.2 124.489315) (end 123.365685 123.655) (width 0.2) (layer "F.Cu") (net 4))
 (segment (start 123.865685 125.155) (end 124.2 124.820685) (width 0.2) (layer "F.Cu") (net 4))
 (segment (start 123.5 131.2) (end 123.5 128.665) (width 0.2) (layer "F.Cu") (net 1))
 (segment (start 123.5 128.665) (end 122.99 128.155) (width 0.2) (layer "F.Cu") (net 1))
 (segment (start 121.73 128.155) (end 122.99 128.155) (width 0.2) (layer "F.Cu") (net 1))
 (segment (start 123.5 126.155) (end 123.5 127.645) (width 0.2) (layer "F.Cu") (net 1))
 (segment (start 123.5 127.645) (end 122.99 128.155) (width 0.2) (layer "F.Cu") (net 1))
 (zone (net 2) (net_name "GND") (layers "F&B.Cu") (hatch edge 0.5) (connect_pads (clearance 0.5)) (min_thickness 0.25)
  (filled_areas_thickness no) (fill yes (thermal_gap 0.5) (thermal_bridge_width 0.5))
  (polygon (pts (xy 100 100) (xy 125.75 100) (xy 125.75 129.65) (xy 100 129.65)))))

